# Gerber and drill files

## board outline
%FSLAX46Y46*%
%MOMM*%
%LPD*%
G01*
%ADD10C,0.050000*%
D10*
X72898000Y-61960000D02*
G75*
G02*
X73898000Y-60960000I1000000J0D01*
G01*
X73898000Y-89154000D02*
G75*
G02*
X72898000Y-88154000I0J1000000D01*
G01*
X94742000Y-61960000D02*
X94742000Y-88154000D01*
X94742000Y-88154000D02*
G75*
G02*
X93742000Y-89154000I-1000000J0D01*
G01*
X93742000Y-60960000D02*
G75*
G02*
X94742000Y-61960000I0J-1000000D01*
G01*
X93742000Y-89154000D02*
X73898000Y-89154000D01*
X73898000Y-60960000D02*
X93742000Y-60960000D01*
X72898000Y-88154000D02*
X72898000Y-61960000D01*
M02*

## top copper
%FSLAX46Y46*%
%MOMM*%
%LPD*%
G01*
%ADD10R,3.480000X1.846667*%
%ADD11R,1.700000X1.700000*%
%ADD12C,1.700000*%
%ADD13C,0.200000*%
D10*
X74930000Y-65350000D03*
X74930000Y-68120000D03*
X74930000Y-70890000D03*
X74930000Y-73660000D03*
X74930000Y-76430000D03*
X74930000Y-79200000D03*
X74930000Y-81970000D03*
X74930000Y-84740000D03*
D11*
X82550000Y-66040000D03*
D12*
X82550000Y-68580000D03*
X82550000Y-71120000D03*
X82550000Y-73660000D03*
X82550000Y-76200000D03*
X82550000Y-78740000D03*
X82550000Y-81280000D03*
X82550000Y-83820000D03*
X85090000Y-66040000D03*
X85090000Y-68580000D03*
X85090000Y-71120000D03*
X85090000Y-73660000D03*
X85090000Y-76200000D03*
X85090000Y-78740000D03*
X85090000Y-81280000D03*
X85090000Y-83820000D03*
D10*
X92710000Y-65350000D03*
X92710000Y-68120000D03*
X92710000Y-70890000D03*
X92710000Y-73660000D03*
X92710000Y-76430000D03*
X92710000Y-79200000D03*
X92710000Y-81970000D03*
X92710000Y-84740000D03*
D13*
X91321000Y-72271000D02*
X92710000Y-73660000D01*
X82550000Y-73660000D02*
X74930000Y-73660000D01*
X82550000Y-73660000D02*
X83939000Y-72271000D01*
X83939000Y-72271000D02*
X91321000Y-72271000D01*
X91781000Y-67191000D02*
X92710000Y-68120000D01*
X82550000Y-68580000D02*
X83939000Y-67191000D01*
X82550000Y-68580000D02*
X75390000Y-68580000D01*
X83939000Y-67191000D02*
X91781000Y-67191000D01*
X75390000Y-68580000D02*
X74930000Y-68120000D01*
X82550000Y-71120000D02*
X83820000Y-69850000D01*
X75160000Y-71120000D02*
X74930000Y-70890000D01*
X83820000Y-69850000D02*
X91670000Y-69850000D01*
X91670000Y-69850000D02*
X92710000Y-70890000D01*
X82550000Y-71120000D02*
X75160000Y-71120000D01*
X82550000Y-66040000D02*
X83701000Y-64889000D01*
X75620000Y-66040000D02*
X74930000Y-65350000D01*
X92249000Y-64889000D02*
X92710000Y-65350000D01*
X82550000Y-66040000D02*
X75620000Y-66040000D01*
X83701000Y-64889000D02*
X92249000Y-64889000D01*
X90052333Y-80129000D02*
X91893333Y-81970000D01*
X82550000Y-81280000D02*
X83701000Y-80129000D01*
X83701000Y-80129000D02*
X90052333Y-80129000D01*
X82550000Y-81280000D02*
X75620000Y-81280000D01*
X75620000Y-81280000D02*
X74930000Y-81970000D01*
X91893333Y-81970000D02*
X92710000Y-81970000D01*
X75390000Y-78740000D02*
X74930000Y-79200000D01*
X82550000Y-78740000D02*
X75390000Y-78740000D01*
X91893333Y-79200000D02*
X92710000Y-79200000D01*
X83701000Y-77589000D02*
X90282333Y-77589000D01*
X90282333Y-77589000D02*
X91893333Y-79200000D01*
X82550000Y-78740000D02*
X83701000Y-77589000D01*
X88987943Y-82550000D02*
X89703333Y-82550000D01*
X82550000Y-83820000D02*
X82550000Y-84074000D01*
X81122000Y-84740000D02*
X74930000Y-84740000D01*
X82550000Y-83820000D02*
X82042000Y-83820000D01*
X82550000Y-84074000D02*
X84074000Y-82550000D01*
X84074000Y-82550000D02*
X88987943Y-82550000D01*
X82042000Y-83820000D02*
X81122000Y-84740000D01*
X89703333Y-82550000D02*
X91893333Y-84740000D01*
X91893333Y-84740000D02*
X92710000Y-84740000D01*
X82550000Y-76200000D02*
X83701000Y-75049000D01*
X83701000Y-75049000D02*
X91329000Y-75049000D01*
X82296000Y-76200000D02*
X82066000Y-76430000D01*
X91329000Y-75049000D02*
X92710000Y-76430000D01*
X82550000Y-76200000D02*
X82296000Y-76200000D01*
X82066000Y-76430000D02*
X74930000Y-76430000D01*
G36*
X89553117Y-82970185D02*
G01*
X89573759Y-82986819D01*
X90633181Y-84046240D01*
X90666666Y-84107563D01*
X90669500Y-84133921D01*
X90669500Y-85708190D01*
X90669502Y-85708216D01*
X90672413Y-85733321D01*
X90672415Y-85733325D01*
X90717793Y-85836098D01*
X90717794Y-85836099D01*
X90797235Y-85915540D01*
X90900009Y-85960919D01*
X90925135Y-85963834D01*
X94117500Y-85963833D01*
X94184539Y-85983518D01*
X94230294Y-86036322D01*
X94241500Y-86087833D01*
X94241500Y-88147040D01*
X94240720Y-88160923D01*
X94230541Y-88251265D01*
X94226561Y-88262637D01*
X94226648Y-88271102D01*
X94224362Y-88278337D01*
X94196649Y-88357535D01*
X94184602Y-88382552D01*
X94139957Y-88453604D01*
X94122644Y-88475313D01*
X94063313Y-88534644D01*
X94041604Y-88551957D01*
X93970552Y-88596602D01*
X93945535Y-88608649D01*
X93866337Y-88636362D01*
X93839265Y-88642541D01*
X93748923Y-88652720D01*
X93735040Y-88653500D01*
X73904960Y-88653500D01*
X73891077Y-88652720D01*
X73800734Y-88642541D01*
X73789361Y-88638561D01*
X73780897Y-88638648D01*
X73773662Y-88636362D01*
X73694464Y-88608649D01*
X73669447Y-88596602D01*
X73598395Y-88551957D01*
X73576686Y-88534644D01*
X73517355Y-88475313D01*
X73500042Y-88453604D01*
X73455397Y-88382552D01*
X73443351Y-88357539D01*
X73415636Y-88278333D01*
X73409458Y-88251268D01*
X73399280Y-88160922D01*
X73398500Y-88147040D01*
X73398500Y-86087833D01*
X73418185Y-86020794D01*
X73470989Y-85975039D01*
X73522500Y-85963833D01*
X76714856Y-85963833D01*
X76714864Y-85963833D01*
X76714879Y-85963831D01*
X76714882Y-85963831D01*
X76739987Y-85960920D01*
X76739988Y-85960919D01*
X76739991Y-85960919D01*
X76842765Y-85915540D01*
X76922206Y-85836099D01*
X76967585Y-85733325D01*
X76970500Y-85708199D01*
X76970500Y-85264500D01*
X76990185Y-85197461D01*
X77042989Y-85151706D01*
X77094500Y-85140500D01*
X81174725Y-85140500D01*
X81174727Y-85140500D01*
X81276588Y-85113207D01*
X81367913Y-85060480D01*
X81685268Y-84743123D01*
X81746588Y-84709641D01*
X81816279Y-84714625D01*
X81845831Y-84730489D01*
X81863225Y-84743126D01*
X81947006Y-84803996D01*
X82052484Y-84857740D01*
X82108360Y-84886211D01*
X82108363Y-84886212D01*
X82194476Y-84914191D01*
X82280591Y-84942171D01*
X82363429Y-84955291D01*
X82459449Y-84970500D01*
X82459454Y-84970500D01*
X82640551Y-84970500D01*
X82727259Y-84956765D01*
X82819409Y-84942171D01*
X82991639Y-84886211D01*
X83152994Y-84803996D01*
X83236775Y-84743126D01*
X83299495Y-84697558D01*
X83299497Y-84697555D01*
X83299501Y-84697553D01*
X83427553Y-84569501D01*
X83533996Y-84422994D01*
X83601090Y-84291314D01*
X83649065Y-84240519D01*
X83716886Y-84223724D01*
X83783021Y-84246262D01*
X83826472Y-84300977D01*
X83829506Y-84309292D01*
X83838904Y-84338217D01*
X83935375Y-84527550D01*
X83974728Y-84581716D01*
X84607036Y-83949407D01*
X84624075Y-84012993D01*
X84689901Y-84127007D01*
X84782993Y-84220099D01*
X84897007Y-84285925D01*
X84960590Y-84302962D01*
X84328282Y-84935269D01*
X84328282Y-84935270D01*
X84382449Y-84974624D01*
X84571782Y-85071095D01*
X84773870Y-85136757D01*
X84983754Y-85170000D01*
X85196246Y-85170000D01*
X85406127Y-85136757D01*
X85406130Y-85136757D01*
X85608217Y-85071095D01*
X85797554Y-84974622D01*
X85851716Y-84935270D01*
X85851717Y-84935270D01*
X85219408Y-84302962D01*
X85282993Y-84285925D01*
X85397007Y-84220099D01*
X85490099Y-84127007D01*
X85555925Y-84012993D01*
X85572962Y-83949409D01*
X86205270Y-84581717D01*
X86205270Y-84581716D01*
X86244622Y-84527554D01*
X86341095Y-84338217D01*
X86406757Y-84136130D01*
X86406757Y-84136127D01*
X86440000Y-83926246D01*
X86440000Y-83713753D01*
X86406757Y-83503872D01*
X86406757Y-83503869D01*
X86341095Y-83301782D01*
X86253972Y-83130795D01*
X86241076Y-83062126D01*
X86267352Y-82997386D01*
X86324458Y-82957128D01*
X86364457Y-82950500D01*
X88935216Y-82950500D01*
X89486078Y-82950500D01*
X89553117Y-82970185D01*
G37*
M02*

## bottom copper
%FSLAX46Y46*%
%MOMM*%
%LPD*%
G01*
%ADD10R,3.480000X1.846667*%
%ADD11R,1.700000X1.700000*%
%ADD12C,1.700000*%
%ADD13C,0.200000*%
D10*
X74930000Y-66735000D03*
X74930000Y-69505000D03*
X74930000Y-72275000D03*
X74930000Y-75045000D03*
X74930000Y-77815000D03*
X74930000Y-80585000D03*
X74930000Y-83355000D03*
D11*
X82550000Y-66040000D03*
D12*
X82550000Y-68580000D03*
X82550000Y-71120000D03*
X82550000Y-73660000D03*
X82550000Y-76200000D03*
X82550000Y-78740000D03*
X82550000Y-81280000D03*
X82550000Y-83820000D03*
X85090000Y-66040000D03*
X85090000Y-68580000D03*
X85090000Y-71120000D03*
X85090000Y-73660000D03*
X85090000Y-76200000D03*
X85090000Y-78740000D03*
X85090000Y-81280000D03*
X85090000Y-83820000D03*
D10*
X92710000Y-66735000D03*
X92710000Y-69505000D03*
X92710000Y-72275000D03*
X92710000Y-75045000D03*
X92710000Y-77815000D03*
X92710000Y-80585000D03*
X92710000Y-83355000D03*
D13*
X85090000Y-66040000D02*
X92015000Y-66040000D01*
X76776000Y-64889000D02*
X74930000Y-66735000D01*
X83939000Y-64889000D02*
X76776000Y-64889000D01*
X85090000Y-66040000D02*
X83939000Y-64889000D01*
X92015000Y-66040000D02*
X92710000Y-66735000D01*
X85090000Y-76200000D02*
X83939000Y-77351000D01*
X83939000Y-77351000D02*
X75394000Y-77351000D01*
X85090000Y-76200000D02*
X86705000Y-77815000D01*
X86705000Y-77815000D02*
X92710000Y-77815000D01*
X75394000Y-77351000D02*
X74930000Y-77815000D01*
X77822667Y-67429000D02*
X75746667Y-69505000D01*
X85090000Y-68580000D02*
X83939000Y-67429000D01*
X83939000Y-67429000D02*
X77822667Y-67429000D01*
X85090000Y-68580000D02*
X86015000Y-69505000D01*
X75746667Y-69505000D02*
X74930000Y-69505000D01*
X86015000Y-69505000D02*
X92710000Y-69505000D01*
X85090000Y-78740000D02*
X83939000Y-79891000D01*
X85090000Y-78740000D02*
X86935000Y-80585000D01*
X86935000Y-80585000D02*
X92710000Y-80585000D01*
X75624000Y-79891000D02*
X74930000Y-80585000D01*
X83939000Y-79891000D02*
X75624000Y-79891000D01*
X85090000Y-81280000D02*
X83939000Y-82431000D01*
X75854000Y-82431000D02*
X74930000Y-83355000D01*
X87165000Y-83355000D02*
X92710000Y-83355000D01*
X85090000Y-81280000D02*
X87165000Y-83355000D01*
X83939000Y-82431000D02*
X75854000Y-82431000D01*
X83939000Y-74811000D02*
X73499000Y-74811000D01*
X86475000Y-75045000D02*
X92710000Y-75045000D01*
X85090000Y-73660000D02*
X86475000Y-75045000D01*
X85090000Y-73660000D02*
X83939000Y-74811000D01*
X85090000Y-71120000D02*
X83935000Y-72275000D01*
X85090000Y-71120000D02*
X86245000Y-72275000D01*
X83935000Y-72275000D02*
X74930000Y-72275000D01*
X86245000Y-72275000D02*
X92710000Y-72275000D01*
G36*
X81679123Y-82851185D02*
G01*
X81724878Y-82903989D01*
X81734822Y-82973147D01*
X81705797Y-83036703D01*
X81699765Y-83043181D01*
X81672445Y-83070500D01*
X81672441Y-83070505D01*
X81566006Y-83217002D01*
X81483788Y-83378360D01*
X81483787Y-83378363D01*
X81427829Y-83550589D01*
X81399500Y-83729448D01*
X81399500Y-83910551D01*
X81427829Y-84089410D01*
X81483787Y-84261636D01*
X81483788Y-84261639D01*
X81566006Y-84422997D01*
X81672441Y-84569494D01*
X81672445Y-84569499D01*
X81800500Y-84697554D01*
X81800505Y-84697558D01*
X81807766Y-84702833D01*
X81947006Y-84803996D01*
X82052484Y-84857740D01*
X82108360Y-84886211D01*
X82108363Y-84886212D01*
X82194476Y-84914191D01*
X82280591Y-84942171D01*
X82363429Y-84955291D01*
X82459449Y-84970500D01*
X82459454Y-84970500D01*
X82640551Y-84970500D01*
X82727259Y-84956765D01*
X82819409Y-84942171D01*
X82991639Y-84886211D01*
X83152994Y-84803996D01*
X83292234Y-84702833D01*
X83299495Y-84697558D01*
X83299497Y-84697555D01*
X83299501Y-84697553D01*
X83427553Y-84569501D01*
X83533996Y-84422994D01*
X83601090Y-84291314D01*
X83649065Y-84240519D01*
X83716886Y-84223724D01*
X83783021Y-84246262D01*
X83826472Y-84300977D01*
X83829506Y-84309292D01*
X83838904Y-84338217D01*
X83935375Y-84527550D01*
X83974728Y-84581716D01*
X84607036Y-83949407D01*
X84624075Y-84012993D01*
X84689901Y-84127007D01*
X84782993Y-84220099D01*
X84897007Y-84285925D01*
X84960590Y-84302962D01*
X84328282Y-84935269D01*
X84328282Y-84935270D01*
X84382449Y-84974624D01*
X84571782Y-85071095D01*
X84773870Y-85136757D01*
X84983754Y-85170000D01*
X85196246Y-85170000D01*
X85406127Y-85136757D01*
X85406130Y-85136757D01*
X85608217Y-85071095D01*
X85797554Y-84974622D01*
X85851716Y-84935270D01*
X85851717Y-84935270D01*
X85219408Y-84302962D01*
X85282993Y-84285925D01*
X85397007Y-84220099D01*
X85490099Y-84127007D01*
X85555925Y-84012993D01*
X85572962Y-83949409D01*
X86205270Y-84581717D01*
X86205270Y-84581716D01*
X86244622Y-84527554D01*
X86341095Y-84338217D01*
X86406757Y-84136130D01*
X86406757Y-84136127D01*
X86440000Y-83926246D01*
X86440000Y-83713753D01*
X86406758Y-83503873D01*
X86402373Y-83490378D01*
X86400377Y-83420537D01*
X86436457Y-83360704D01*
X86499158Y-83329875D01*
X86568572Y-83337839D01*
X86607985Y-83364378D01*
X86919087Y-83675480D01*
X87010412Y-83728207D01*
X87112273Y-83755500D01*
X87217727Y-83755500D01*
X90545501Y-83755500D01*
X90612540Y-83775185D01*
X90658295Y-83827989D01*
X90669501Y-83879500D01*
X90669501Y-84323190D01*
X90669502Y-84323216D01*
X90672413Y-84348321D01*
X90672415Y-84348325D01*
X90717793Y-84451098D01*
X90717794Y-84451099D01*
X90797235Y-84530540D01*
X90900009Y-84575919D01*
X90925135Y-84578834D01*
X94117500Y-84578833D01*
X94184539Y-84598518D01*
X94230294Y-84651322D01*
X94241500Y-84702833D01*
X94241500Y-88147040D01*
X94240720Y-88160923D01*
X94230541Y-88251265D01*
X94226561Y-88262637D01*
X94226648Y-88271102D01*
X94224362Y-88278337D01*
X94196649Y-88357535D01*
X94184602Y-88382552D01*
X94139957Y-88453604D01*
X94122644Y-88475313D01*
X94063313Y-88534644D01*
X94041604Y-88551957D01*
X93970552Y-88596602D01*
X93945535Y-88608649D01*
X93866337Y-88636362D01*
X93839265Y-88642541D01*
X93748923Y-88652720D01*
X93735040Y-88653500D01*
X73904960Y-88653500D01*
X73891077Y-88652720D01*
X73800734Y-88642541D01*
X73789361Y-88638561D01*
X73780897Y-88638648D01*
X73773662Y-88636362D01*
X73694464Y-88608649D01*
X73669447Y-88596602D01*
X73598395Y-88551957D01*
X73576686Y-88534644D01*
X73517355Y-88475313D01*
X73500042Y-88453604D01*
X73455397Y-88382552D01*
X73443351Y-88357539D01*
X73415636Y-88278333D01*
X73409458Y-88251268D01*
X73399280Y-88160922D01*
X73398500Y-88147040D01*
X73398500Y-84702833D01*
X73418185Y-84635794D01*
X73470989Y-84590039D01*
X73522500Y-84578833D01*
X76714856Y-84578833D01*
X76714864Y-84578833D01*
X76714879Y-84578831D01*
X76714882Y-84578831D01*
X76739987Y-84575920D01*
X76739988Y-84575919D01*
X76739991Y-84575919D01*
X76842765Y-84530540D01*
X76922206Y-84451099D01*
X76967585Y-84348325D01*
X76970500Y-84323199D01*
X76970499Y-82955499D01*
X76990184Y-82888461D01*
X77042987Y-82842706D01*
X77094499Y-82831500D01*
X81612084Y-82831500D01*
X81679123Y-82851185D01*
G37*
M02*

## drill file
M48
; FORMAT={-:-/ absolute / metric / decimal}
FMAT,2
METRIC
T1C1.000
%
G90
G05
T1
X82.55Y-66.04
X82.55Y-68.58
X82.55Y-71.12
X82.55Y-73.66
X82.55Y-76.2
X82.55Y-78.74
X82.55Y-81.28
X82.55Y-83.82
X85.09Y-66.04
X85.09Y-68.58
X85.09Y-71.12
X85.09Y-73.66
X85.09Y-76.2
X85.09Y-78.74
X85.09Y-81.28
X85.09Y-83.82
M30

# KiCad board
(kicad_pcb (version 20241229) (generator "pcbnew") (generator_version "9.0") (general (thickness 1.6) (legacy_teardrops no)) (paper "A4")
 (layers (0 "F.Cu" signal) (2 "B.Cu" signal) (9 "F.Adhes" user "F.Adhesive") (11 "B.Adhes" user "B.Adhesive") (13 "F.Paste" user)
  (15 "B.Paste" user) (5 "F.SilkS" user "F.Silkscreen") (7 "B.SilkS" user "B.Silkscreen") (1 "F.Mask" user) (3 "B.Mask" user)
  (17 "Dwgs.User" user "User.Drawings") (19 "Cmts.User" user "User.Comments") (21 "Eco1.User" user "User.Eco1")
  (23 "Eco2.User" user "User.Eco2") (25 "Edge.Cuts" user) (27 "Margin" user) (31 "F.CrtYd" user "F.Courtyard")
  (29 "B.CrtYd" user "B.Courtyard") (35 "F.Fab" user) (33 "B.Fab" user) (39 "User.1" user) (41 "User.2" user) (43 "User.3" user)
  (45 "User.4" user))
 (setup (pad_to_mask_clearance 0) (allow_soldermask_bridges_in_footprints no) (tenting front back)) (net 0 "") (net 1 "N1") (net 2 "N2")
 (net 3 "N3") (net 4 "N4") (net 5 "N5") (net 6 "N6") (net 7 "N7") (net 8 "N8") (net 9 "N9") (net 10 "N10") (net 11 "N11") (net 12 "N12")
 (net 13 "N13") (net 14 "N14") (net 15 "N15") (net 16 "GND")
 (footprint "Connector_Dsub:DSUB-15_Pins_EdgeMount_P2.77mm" (layer "F.Cu") (at 74.93 75.045 -90)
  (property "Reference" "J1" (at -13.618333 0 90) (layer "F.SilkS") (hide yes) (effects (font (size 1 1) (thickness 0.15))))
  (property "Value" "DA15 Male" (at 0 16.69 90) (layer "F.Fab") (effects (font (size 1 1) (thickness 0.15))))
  (pad "1" smd rect (at -9.695 0 270) (size 1.846667 3.48) (layers "F.Cu" "F.Mask" "F.Paste") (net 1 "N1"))
  (pad "2" smd rect (at -6.925 0 270) (size 1.846667 3.48) (layers "F.Cu" "F.Mask" "F.Paste") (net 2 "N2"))
  (pad "3" smd rect (at -4.155 0 270) (size 1.846667 3.48) (layers "F.Cu" "F.Mask" "F.Paste") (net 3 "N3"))
  (pad "4" smd rect (at -1.385 0 270) (size 1.846667 3.48) (layers "F.Cu" "F.Mask" "F.Paste") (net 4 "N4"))
  (pad "5" smd rect (at 1.385 0 270) (size 1.846667 3.48) (layers "F.Cu" "F.Mask" "F.Paste") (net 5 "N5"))
  (pad "6" smd rect (at 4.155 0 270) (size 1.846667 3.48) (layers "F.Cu" "F.Mask" "F.Paste") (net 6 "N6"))
  (pad "7" smd rect (at 6.925 0 270) (size 1.846667 3.48) (layers "F.Cu" "F.Mask" "F.Paste") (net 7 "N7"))
  (pad "8" smd rect (at 9.695 0 270) (size 1.846667 3.48) (layers "F.Cu" "F.Mask" "F.Paste") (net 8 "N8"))
  (pad "9" smd rect (at -8.31 0 270) (size 1.846667 3.48) (layers "B.Cu" "B.Mask" "B.Paste") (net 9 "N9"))
  (pad "10" smd rect (at -5.54 0 270) (size 1.846667 3.48) (layers "B.Cu" "B.Mask" "B.Paste") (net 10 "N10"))
  (pad "11" smd rect (at -2.77 0 270) (size 1.846667 3.48) (layers "B.Cu" "B.Mask" "B.Paste") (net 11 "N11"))
  (pad "12" smd rect (at 0 0 270) (size 1.846667 3.48) (layers "B.Cu" "B.Mask" "B.Paste") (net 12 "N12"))
  (pad "13" smd rect (at 2.77 0 270) (size 1.846667 3.48) (layers "B.Cu" "B.Mask" "B.Paste") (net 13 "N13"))
  (pad "14" smd rect (at 5.54 0 270) (size 1.846667 3.48) (layers "B.Cu" "B.Mask" "B.Paste") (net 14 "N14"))
  (pad "15" smd rect (at 8.31 0 270) (size 1.846667 3.48) (layers "B.Cu" "B.Mask" "B.Paste") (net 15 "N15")))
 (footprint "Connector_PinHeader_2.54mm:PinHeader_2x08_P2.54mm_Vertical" (layer "F.Cu") (at 82.55 66.04)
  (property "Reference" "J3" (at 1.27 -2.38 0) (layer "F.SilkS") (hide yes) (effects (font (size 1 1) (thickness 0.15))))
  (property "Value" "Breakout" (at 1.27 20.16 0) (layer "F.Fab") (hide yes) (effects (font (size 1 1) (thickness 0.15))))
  (pad "1" thru_hole rect (at 0 0) (size 1.7 1.7) (drill 1) (layers "*.Cu" "*.Mask") (remove_unused_layers no) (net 1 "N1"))
  (pad "2" thru_hole circle (at 0 2.54) (size 1.7 1.7) (drill 1) (layers "*.Cu" "*.Mask") (remove_unused_layers no) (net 2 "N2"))
  (pad "3" thru_hole circle (at 0 5.08) (size 1.7 1.7) (drill 1) (layers "*.Cu" "*.Mask") (remove_unused_layers no) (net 3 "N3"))
  (pad "4" thru_hole circle (at 0 7.62) (size 1.7 1.7) (drill 1) (layers "*.Cu" "*.Mask") (remove_unused_layers no) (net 4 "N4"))
  (pad "5" thru_hole circle (at 0 10.16) (size 1.7 1.7) (drill 1) (layers "*.Cu" "*.Mask") (remove_unused_layers no) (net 5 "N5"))
  (pad "6" thru_hole circle (at 0 12.7) (size 1.7 1.7) (drill 1) (layers "*.Cu" "*.Mask") (remove_unused_layers no) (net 6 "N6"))
  (pad "7" thru_hole circle (at 0 15.24) (size 1.7 1.7) (drill 1) (layers "*.Cu" "*.Mask") (remove_unused_layers no) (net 7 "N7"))
  (pad "8" thru_hole circle (at 0 17.78) (size 1.7 1.7) (drill 1) (layers "*.Cu" "*.Mask") (remove_unused_layers no) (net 8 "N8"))
  (pad "9" thru_hole circle (at 2.54 0) (size 1.7 1.7) (drill 1) (layers "*.Cu" "*.Mask") (remove_unused_layers no) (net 9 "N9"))
  (pad "10" thru_hole circle (at 2.54 2.54) (size 1.7 1.7) (drill 1) (layers "*.Cu" "*.Mask") (remove_unused_layers no) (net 10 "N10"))
  (pad "11" thru_hole circle (at 2.54 5.08) (size 1.7 1.7) (drill 1) (layers "*.Cu" "*.Mask") (remove_unused_layers no) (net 11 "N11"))
  (pad "12" thru_hole circle (at 2.54 7.62) (size 1.7 1.7) (drill 1) (layers "*.Cu" "*.Mask") (remove_unused_layers no) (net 12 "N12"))
  (pad "13" thru_hole circle (at 2.54 10.16) (size 1.7 1.7) (drill 1) (layers "*.Cu" "*.Mask") (remove_unused_layers no) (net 13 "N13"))
  (pad "14" thru_hole circle (at 2.54 12.7) (size 1.7 1.7) (drill 1) (layers "*.Cu" "*.Mask") (remove_unused_layers no) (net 14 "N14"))
  (pad "15" thru_hole circle (at 2.54 15.24) (size 1.7 1.7) (drill 1) (layers "*.Cu" "*.Mask") (remove_unused_layers no) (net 15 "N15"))
  (pad "16" thru_hole circle (at 2.54 17.78) (size 1.7 1.7) (drill 1) (layers "*.Cu" "*.Mask") (remove_unused_layers no) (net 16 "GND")))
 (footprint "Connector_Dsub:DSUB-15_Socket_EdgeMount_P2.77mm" (layer "F.Cu") (at 92.71 75.045 90)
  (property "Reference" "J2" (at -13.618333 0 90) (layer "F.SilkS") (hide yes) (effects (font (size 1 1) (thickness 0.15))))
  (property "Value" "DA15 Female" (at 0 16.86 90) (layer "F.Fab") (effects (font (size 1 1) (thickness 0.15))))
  (pad "1" smd rect (at 9.695 0 90) (size 1.846667 3.48) (layers "F.Cu" "F.Mask" "F.Paste") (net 1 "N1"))
  (pad "2" smd rect (at 6.925 0 90) (size 1.846667 3.48) (layers "F.Cu" "F.Mask" "F.Paste") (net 2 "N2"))
  (pad "3" smd rect (at 4.155 0 90) (size 1.846667 3.48) (layers "F.Cu" "F.Mask" "F.Paste") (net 3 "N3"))
  (pad "4" smd rect (at 1.385 0 90) (size 1.846667 3.48) (layers "F.Cu" "F.Mask" "F.Paste") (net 4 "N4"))
  (pad "5" smd rect (at -1.385 0 90) (size 1.846667 3.48) (layers "F.Cu" "F.Mask" "F.Paste") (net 5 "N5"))
  (pad "6" smd rect (at -4.155 0 90) (size 1.846667 3.48) (layers "F.Cu" "F.Mask" "F.Paste") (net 6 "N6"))
  (pad "7" smd rect (at -6.925 0 90) (size 1.846667 3.48) (layers "F.Cu" "F.Mask" "F.Paste") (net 7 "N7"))
  (pad "8" smd rect (at -9.695 0 90) (size 1.846667 3.48) (layers "F.Cu" "F.Mask" "F.Paste") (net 8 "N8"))
  (pad "9" smd rect (at 8.31 0 90) (size 1.846667 3.48) (layers "B.Cu" "B.Mask" "B.Paste") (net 9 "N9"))
  (pad "10" smd rect (at 5.54 0 90) (size 1.846667 3.48) (layers "B.Cu" "B.Mask" "B.Paste") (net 10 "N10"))
  (pad "11" smd rect (at 2.77 0 90) (size 1.846667 3.48) (layers "B.Cu" "B.Mask" "B.Paste") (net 11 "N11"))
  (pad "12" smd rect (at 0 0 90) (size 1.846667 3.48) (layers "B.Cu" "B.Mask" "B.Paste") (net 12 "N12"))
  (pad "13" smd rect (at -2.77 0 90) (size 1.846667 3.48) (layers "B.Cu" "B.Mask" "B.Paste") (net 13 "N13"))
  (pad "14" smd rect (at -5.54 0 90) (size 1.846667 3.48) (layers "B.Cu" "B.Mask" "B.Paste") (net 14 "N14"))
  (pad "15" smd rect (at -8.31 0 90) (size 1.846667 3.48) (layers "B.Cu" "B.Mask" "B.Paste") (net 15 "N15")))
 (gr_arc (start 72.898 61.96) (mid 73.190893 61.252893) (end 73.898 60.96) (stroke (width 0.05) (type default)) (layer "Edge.Cuts"))
 (gr_arc (start 73.898 89.154) (mid 73.190893 88.861107) (end 72.898 88.154) (stroke (width 0.05) (type default)) (layer "Edge.Cuts"))
 (gr_line (start 94.742 61.96) (end 94.742 88.154) (stroke (width 0.05) (type default)) (layer "Edge.Cuts"))
 (gr_arc (start 94.742 88.154) (mid 94.449107 88.861107) (end 93.742 89.154) (stroke (width 0.05) (type default)) (layer "Edge.Cuts"))
 (gr_arc (start 93.742 60.96) (mid 94.449107 61.252893) (end 94.742 61.96) (stroke (width 0.05) (type default)) (layer "Edge.Cuts"))
 (gr_line (start 93.742 89.154) (end 73.898 89.154) (stroke (width 0.05) (type default)) (layer "Edge.Cuts"))
 (gr_line (start 73.898 60.96) (end 93.742 60.96) (stroke (width 0.05) (type default)) (layer "Edge.Cuts"))
 (gr_line (start 72.898 88.154) (end 72.898 61.96) (stroke (width 0.05) (type default)) (layer "Edge.Cuts"))
 (segment (start 85.09 66.04) (end 92.015 66.04) (width 0.2) (layer "B.Cu") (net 9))
 (segment (start 76.776 64.889) (end 74.93 66.735) (width 0.2) (layer "B.Cu") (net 9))
 (segment (start 83.939 64.889) (end 76.776 64.889) (width 0.2) (layer "B.Cu") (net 9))
 (segment (start 85.09 66.04) (end 83.939 64.889) (width 0.2) (layer "B.Cu") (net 9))
 (segment (start 92.015 66.04) (end 92.71 66.735) (width 0.2) (layer "B.Cu") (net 9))
 (segment (start 85.09 76.2) (end 83.939 77.351) (width 0.2) (layer "B.Cu") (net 13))
 (segment (start 83.939 77.351) (end 75.394 77.351) (width 0.2) (layer "B.Cu") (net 13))
 (segment (start 85.09 76.2) (end 86.705 77.815) (width 0.2) (layer "B.Cu") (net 13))
 (segment (start 86.705 77.815) (end 92.71 77.815) (width 0.2) (layer "B.Cu") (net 13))
 (segment (start 75.394 77.351) (end 74.93 77.815) (width 0.2) (layer "B.Cu") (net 13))
 (segment (start 91.321 72.271) (end 92.71 73.66) (width 0.2) (layer "F.Cu") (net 4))
 (segment (start 82.55 73.66) (end 74.93 73.66) (width 0.2) (layer "F.Cu") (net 4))
 (segment (start 82.55 73.66) (end 83.939 72.271) (width 0.2) (layer "F.Cu") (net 4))
 (segment (start 83.939 72.271) (end 91.321 72.271) (width 0.2) (layer "F.Cu") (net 4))
 (segment (start 77.822667 67.429) (end 75.746667 69.505) (width 0.2) (layer "B.Cu") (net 10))
 (segment (start 85.09 68.58) (end 83.939 67.429) (width 0.2) (layer "B.Cu") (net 10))
 (segment (start 83.939 67.429) (end 77.822667 67.429) (width 0.2) (layer "B.Cu") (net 10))
 (segment (start 85.09 68.58) (end 86.015 69.505) (width 0.2) (layer "B.Cu") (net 10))
 (segment (start 75.746667 69.505) (end 74.93 69.505) (width 0.2) (layer "B.Cu") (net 10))
 (segment (start 86.015 69.505) (end 92.71 69.505) (width 0.2) (layer "B.Cu") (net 10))
 (segment (start 91.781 67.191) (end 92.71 68.12) (width 0.2) (layer "F.Cu") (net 2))
 (segment (start 82.55 68.58) (end 83.939 67.191) (width 0.2) (layer "F.Cu") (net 2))
 (segment (start 82.55 68.58) (end 75.39 68.58) (width 0.2) (layer "F.Cu") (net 2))
 (segment (start 83.939 67.191) (end 91.781 67.191) (width 0.2) (layer "F.Cu") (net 2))
 (segment (start 75.39 68.58) (end 74.93 68.12) (width 0.2) (layer "F.Cu") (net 2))
 (segment (start 82.55 71.12) (end 83.82 69.85) (width 0.2) (layer "F.Cu") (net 3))
 (segment (start 75.16 71.12) (end 74.93 70.89) (width 0.2) (layer "F.Cu") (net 3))
 (segment (start 83.82 69.85) (end 91.67 69.85) (width 0.2) (layer "F.Cu") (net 3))
 (segment (start 91.67 69.85) (end 92.71 70.89) (width 0.2) (layer "F.Cu") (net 3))
 (segment (start 82.55 71.12) (end 75.16 71.12) (width 0.2) (layer "F.Cu") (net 3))
 (segment (start 85.09 78.74) (end 83.939 79.891) (width 0.2) (layer "B.Cu") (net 14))
 (segment (start 85.09 78.74) (end 86.935 80.585) (width 0.2) (layer "B.Cu") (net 14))
 (segment (start 86.935 80.585) (end 92.71 80.585) (width 0.2) (layer "B.Cu") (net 14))
 (segment (start 75.624 79.891) (end 74.93 80.585) (width 0.2) (layer "B.Cu") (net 14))
 (segment (start 83.939 79.891) (end 75.624 79.891) (width 0.2) (layer "B.Cu") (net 14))
 (segment (start 82.55 66.04) (end 83.701 64.889) (width 0.2) (layer "F.Cu") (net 1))
 (segment (start 75.62 66.04) (end 74.93 65.35) (width 0.2) (layer "F.Cu") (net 1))
 (segment (start 92.249 64.889) (end 92.71 65.35) (width 0.2) (layer "F.Cu") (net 1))
 (segment (start 82.55 66.04) (end 75.62 66.04) (width 0.2) (layer "F.Cu") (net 1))
 (segment (start 83.701 64.889) (end 92.249 64.889) (width 0.2) (layer "F.Cu") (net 1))
 (segment (start 90.052333 80.129) (end 91.893333 81.97) (width 0.2) (layer "F.Cu") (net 7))
 (segment (start 82.55 81.28) (end 83.701 80.129) (width 0.2) (layer "F.Cu") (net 7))
 (segment (start 83.701 80.129) (end 90.052333 80.129) (width 0.2) (layer "F.Cu") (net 7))
 (segment (start 82.55 81.28) (end 75.62 81.28) (width 0.2) (layer "F.Cu") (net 7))
 (segment (start 75.62 81.28) (end 74.93 81.97) (width 0.2) (layer "F.Cu") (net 7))
 (segment (start 91.893333 81.97) (end 92.71 81.97) (width 0.2) (layer "F.Cu") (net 7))
 (segment (start 85.09 81.28) (end 83.939 82.431) (width 0.2) (layer "B.Cu") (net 15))
 (segment (start 75.854 82.431) (end 74.93 83.355) (width 0.2) (layer "B.Cu") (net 15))
 (segment (start 87.165 83.355) (end 92.71 83.355) (width 0.2) (layer "B.Cu") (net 15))
 (segment (start 85.09 81.28) (end 87.165 83.355) (width 0.2) (layer "B.Cu") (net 15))
 (segment (start 83.939 82.431) (end 75.854 82.431) (width 0.2) (layer "B.Cu") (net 15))
 (segment (start 75.39 78.74) (end 74.93 79.2) (width 0.2) (layer "F.Cu") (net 6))
 (segment (start 82.55 78.74) (end 75.39 78.74) (width 0.2) (layer "F.Cu") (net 6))
 (segment (start 91.893333 79.2) (end 92.71 79.2) (width 0.2) (layer "F.Cu") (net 6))
 (segment (start 83.701 77.589) (end 90.282333 77.589) (width 0.2) (layer "F.Cu") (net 6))
 (segment (start 90.282333 77.589) (end 91.893333 79.2) (width 0.2) (layer "F.Cu") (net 6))
 (segment (start 82.55 78.74) (end 83.701 77.589) (width 0.2) (layer "F.Cu") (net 6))
 (segment (start 83.939 74.811) (end 73.499 74.811) (width 0.2) (layer "B.Cu") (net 12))
 (segment (start 86.475 75.045) (end 92.71 75.045) (width 0.2) (layer "B.Cu") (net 12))
 (segment (start 85.09 73.66) (end 86.475 75.045) (width 0.2) (layer "B.Cu") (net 12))
 (segment (start 85.09 73.66) (end 83.939 74.811) (width 0.2) (layer "B.Cu") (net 12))
 (segment (start 88.987943 82.55) (end 89.703333 82.55) (width 0.2) (layer "F.Cu") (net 8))
 (segment (start 82.55 83.82) (end 82.55 84.074) (width 0.2) (layer "F.Cu") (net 8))
 (segment (start 81.122 84.74) (end 74.93 84.74) (width 0.2) (layer "F.Cu") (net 8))
 (segment (start 82.55 83.82) (end 82.042 83.82) (width 0.2) (layer "F.Cu") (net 8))
 (segment (start 82.55 84.074) (end 84.074 82.55) (width 0.2) (layer "F.Cu") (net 8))
 (segment (start 84.074 82.55) (end 88.987943 82.55) (width 0.2) (layer "F.Cu") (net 8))
 (segment (start 82.042 83.82) (end 81.122 84.74) (width 0.2) (layer "F.Cu") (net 8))
 (segment (start 89.703333 82.55) (end 91.893333 84.74) (width 0.2) (layer "F.Cu") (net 8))
 (segment (start 91.893333 84.74) (end 92.71 84.74) (width 0.2) (layer "F.Cu") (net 8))
 (segment (start 82.55 76.2) (end 83.701 75.049) (width 0.2) (layer "F.Cu") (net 5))
 (segment (start 83.701 75.049) (end 91.329 75.049) (width 0.2) (layer "F.Cu") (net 5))
 (segment (start 82.296 76.2) (end 82.066 76.43) (width 0.2) (layer "F.Cu") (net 5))
 (segment (start 91.329 75.049) (end 92.71 76.43) (width 0.2) (layer "F.Cu") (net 5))
 (segment (start 82.55 76.2) (end 82.296 76.2) (width 0.2) (layer "F.Cu") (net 5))
 (segment (start 82.066 76.43) (end 74.93 76.43) (width 0.2) (layer "F.Cu") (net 5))
 (segment (start 85.09 71.12) (end 83.935 72.275) (width 0.2) (layer "B.Cu") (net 11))
 (segment (start 85.09 71.12) (end 86.245 72.275) (width 0.2) (layer "B.Cu") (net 11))
 (segment (start 83.935 72.275) (end 74.93 72.275) (width 0.2) (layer "B.Cu") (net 11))
 (segment (start 86.245 72.275) (end 92.71 72.275) (width 0.2) (layer "B.Cu") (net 11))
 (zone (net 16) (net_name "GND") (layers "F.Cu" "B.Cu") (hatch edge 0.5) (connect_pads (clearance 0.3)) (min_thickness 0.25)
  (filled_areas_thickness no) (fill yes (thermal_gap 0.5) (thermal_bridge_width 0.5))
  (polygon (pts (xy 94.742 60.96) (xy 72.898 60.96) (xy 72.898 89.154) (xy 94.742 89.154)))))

